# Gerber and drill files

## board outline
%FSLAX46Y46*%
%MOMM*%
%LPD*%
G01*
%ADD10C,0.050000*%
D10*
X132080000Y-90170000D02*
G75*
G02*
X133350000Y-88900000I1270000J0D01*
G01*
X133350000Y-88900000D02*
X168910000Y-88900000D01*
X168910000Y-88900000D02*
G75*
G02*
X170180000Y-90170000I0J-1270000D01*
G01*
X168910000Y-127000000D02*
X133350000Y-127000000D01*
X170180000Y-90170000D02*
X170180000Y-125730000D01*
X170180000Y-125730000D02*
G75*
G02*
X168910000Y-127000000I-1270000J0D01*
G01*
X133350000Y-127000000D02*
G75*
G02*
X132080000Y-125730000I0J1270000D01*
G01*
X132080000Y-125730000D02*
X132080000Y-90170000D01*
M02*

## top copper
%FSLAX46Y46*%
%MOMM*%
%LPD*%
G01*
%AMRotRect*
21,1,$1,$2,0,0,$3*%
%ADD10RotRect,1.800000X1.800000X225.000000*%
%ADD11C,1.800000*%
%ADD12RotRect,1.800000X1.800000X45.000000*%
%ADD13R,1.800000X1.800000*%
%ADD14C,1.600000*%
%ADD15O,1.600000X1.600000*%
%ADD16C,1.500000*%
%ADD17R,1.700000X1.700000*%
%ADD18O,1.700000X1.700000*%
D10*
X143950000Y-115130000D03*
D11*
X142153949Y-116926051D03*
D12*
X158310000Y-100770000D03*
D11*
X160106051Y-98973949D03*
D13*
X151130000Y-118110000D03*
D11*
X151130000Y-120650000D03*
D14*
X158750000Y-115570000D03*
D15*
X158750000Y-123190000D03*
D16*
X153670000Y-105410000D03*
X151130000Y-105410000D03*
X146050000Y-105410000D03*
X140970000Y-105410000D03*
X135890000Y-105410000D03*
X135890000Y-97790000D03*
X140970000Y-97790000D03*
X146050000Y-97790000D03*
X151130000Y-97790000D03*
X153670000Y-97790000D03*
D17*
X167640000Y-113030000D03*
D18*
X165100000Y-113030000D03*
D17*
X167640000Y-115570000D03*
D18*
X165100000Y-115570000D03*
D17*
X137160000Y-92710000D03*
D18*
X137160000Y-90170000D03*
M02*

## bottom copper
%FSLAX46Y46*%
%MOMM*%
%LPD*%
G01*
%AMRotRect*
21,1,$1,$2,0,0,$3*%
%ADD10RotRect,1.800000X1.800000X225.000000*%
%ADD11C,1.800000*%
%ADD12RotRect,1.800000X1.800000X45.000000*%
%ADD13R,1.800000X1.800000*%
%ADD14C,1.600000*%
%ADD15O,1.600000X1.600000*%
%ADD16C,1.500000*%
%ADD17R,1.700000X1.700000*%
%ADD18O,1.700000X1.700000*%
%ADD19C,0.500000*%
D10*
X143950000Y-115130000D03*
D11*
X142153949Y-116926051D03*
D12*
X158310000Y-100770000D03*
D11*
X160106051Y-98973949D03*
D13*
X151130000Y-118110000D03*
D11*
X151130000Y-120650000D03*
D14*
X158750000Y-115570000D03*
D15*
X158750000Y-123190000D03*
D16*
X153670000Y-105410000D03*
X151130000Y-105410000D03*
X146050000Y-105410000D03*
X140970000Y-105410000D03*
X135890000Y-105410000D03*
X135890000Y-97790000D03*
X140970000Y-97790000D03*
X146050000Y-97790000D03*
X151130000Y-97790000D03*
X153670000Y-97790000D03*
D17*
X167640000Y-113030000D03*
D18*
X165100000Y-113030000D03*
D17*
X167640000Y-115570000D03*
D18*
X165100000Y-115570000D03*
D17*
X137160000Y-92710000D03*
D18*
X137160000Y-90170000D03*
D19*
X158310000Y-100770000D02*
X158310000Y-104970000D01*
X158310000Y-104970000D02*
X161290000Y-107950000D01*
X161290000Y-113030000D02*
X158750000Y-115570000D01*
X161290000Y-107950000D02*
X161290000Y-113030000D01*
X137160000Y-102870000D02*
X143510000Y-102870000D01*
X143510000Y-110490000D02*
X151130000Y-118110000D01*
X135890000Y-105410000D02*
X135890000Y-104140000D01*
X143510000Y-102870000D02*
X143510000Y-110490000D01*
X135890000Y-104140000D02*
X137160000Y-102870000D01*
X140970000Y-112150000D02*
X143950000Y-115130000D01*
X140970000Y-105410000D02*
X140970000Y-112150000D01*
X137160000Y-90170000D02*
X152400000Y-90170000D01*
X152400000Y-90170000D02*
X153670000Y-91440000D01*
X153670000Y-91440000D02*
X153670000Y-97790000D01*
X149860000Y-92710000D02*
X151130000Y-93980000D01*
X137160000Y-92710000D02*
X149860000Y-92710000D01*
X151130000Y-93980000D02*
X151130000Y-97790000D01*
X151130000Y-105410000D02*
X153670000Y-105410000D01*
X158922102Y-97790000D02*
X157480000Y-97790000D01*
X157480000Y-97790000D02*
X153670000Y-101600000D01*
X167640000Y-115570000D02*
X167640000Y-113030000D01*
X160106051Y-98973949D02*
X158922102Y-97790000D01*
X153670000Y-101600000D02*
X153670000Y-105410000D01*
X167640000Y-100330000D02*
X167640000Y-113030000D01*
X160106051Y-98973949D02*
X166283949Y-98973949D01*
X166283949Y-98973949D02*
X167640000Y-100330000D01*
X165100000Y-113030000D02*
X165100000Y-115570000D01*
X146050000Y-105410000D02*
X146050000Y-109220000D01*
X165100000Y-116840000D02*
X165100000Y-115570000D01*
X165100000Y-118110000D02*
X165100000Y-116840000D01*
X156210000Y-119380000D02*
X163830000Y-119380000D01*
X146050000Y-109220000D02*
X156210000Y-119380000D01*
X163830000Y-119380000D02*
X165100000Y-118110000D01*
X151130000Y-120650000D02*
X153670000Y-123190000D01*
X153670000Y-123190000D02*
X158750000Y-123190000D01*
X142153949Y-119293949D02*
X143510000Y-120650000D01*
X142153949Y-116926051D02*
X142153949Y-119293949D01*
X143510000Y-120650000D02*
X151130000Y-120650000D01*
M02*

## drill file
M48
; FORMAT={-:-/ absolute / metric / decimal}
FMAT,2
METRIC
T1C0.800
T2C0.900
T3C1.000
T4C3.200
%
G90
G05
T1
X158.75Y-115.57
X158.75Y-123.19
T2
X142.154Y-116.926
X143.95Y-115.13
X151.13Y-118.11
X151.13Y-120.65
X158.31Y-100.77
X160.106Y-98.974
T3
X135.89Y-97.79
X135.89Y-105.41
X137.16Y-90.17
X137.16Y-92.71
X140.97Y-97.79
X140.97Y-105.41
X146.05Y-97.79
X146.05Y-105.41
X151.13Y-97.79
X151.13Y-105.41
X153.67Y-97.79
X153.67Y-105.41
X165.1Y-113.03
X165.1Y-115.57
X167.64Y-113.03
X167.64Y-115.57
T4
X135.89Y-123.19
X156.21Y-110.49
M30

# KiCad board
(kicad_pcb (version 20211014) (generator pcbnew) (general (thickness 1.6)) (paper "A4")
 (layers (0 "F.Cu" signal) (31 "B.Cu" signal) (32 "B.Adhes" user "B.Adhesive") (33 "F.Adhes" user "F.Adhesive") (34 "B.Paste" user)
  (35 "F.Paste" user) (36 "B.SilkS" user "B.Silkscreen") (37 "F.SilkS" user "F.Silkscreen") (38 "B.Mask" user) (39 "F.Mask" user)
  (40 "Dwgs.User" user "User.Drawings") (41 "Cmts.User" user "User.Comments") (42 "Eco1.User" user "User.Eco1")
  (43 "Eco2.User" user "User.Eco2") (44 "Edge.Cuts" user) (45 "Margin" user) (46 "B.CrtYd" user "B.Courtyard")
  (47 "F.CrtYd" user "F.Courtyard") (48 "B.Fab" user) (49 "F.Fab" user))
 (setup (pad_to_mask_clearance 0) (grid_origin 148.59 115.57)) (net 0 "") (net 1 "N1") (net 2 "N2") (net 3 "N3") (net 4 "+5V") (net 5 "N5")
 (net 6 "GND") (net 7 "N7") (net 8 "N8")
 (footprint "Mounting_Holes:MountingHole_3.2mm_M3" (layer "F.Cu") (at 156.21 110.49 -90)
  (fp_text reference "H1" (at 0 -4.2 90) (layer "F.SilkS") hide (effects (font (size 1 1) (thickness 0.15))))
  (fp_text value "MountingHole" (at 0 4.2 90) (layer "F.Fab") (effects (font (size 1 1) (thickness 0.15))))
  (pad "" np_thru_hole circle locked (at 0 0 270) (size 3.2 3.2) (drill 3.2) (layers *.Cu *.Mask) (thermal_gap 2)))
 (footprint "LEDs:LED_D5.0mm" (layer "F.Cu") (at 143.95 115.13 -135)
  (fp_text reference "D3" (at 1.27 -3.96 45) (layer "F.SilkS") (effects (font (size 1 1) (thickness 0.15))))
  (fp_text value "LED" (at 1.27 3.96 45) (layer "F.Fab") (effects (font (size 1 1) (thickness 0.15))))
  (pad "1" thru_hole rect locked (at 0 0 225) (size 1.8 1.8) (drill 0.9) (layers *.Cu *.Mask) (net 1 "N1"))
  (pad "2" thru_hole circle locked (at 2.54 0 225) (size 1.8 1.8) (drill 0.9) (layers *.Cu *.Mask) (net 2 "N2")))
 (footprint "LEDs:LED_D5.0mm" (layer "F.Cu") (at 158.31 100.77 45)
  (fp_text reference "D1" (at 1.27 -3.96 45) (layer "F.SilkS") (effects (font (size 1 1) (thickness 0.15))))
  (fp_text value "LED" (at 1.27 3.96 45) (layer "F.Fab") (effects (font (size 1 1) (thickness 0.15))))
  (pad "1" thru_hole rect locked (at 0 0 45) (size 1.8 1.8) (drill 0.9) (layers *.Cu *.Mask) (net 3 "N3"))
  (pad "2" thru_hole circle locked (at 2.54 0 45) (size 1.8 1.8) (drill 0.9) (layers *.Cu *.Mask) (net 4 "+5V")))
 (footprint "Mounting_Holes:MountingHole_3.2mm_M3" (layer "F.Cu") (at 135.89 123.19 -90)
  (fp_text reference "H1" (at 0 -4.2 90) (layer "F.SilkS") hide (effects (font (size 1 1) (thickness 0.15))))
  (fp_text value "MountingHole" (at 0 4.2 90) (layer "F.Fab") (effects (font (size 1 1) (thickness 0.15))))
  (pad "" np_thru_hole circle locked (at 0 0 270) (size 3.2 3.2) (drill 3.2) (layers *.Cu *.Mask) (thermal_gap 2)))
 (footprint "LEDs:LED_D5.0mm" (layer "F.Cu") (at 151.13 118.11 -90)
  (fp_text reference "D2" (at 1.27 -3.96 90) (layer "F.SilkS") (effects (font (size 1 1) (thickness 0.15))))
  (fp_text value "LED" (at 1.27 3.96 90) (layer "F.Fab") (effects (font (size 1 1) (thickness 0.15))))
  (pad "1" thru_hole rect locked (at 0 0 270) (size 1.8 1.8) (drill 0.9) (layers *.Cu *.Mask) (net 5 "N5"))
  (pad "2" thru_hole circle locked (at 2.54 0 270) (size 1.8 1.8) (drill 0.9) (layers *.Cu *.Mask) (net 2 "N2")))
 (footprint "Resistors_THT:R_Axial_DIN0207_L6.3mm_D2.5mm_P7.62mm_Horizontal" (layer "F.Cu") (at 158.75 115.57 -90)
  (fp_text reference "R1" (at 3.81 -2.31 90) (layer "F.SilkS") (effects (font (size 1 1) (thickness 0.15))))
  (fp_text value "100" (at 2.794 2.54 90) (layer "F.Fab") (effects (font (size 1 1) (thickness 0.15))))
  (pad "1" thru_hole circle locked (at 0 0 270) (size 1.6 1.6) (drill 0.8) (layers *.Cu *.Mask) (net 3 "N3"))
  (pad "2" thru_hole oval locked (at 7.62 0 270) (size 1.6 1.6) (drill 0.8) (layers *.Cu *.Mask) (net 2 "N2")))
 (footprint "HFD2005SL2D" (layer "B.Cu") (at 153.67 105.41 180)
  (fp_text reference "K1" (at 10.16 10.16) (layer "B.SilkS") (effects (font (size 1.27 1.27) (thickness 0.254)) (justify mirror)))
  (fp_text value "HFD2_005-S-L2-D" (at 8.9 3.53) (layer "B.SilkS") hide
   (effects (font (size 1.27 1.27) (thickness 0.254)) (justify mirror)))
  (pad "1" thru_hole circle locked (at 0 0 90) (size 1.5 1.5) (drill 1) (layers *.Cu *.Mask "B.SilkS") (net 4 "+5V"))
  (pad "2" thru_hole circle locked (at 2.54 0 90) (size 1.5 1.5) (drill 1) (layers *.Cu *.Mask "B.SilkS") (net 4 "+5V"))
  (pad "4" thru_hole circle locked (at 7.62 0 90) (size 1.5 1.5) (drill 1) (layers *.Cu *.Mask "B.SilkS") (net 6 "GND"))
  (pad "6" thru_hole circle locked (at 12.7 0 90) (size 1.5 1.5) (drill 1) (layers *.Cu *.Mask "B.SilkS") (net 1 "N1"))
  (pad "8" thru_hole circle locked (at 17.78 0 90) (size 1.5 1.5) (drill 1) (layers *.Cu *.Mask "B.SilkS") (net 5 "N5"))
  (pad "9" thru_hole circle locked (at 17.78 7.62 90) (size 1.5 1.5) (drill 1) (layers *.Cu *.Mask "B.SilkS"))
  (pad "11" thru_hole circle locked (at 12.7 7.62 90) (size 1.5 1.5) (drill 1) (layers *.Cu *.Mask "B.SilkS"))
  (pad "13" thru_hole circle locked (at 7.62 7.62 90) (size 1.5 1.5) (drill 1) (layers *.Cu *.Mask "B.SilkS"))
  (pad "15" thru_hole circle locked (at 2.54 7.62 90) (size 1.5 1.5) (drill 1) (layers *.Cu *.Mask "B.SilkS") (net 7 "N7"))
  (pad "16" thru_hole circle locked (at 0 7.62 90) (size 1.5 1.5) (drill 1) (layers *.Cu *.Mask "B.SilkS") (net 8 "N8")))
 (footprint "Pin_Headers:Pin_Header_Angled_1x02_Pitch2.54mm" (layer "B.Cu") (at 167.64 113.03 90)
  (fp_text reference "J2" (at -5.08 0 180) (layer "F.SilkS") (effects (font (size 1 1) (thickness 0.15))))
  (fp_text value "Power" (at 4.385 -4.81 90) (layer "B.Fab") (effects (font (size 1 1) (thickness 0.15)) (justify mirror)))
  (pad "1" thru_hole rect locked (at 0 0 90) (size 1.7 1.7) (drill 1) (layers *.Cu *.Mask) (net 4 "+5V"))
  (pad "2" thru_hole oval locked (at 0 -2.54 90) (size 1.7 1.7) (drill 1) (layers *.Cu *.Mask) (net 6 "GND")))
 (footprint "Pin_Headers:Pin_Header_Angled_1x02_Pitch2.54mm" (layer "B.Cu") (at 167.64 115.57 90)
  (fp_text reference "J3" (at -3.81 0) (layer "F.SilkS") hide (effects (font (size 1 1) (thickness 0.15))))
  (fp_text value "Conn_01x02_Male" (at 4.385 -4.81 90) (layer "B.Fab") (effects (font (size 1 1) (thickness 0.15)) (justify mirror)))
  (pad "1" thru_hole rect locked (at 0 0 90) (size 1.7 1.7) (drill 1) (layers *.Cu *.Mask) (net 4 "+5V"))
  (pad "2" thru_hole oval locked (at 0 -2.54 90) (size 1.7 1.7) (drill 1) (layers *.Cu *.Mask) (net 6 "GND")))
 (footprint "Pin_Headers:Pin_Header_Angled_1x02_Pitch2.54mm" (layer "B.Cu") (at 137.16 92.71)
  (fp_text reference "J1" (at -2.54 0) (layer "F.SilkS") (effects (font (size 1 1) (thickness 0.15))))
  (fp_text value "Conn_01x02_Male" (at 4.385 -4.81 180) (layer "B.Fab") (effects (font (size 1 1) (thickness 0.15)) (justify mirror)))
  (pad "1" thru_hole rect locked (at 0 0) (size 1.7 1.7) (drill 1) (layers *.Cu *.Mask) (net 7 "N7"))
  (pad "2" thru_hole oval locked (at 0 -2.54) (size 1.7 1.7) (drill 1) (layers *.Cu *.Mask) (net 8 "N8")))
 (gr_arc (start 132.08 90.17) (mid 132.451974 89.271974) (end 133.35 88.9) (layer "Edge.Cuts") (width 0.05))
 (gr_line (start 133.35 88.9) (end 168.91 88.9) (layer "Edge.Cuts") (width 0.05))
 (gr_arc (start 168.91 88.9) (mid 169.808026 89.271974) (end 170.18 90.17) (layer "Edge.Cuts") (width 0.05))
 (gr_line (start 168.91 127) (end 133.35 127) (layer "Edge.Cuts") (width 0.05))
 (gr_line (start 170.18 90.17) (end 170.18 125.73) (layer "Edge.Cuts") (width 0.05))
 (gr_arc (start 170.18 125.73) (mid 169.808026 126.628026) (end 168.91 127) (layer "Edge.Cuts") (width 0.05))
 (gr_arc (start 133.35 127) (mid 132.451974 126.628026) (end 132.08 125.73) (layer "Edge.Cuts") (width 0.05))
 (gr_line (start 132.08 125.73) (end 132.08 90.17) (layer "Edge.Cuts") (width 0.05))
 (segment (start 158.31 100.77) (end 158.31 104.97) (width 0.5) (layer "B.Cu") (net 3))
 (segment (start 158.31 104.97) (end 161.29 107.95) (width 0.5) (layer "B.Cu") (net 3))
 (segment (start 161.29 113.03) (end 158.75 115.57) (width 0.5) (layer "B.Cu") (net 3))
 (segment (start 161.29 107.95) (end 161.29 113.03) (width 0.5) (layer "B.Cu") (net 3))
 (segment (start 137.16 102.87) (end 143.51 102.87) (width 0.5) (layer "B.Cu") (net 5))
 (segment (start 143.51 110.49) (end 151.13 118.11) (width 0.5) (layer "B.Cu") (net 5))
 (segment (start 135.89 105.41) (end 135.89 104.14) (width 0.5) (layer "B.Cu") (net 5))
 (segment (start 143.51 102.87) (end 143.51 110.49) (width 0.5) (layer "B.Cu") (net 5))
 (segment (start 135.89 104.14) (end 137.16 102.87) (width 0.5) (layer "B.Cu") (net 5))
 (segment (start 140.97 112.15) (end 143.95 115.13) (width 0.5) (layer "B.Cu") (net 1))
 (segment (start 140.97 105.41) (end 140.97 112.15) (width 0.5) (layer "B.Cu") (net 1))
 (segment (start 137.16 90.17) (end 152.4 90.17) (width 0.5) (layer "B.Cu") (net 8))
 (segment (start 152.4 90.17) (end 153.67 91.44) (width 0.5) (layer "B.Cu") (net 8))
 (segment (start 153.67 91.44) (end 153.67 97.79) (width 0.5) (layer "B.Cu") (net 8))
 (segment (start 149.86 92.71) (end 151.13 93.98) (width 0.5) (layer "B.Cu") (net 7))
 (segment (start 137.16 92.71) (end 149.86 92.71) (width 0.5) (layer "B.Cu") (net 7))
 (segment (start 151.13 93.98) (end 151.13 97.79) (width 0.5) (layer "B.Cu") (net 7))
 (segment (start 151.13 105.41) (end 153.67 105.41) (width 0.5) (layer "B.Cu") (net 4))
 (segment (start 158.922102 97.79) (end 157.48 97.79) (width 0.5) (layer "B.Cu") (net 4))
 (segment (start 157.48 97.79) (end 153.67 101.6) (width 0.5) (layer "B.Cu") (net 4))
 (segment (start 167.64 115.57) (end 167.64 113.03) (width 0.5) (layer "B.Cu") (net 4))
 (segment (start 160.106051 98.973949) (end 158.922102 97.79) (width 0.5) (layer "B.Cu") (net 4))
 (segment (start 153.67 101.6) (end 153.67 105.41) (width 0.5) (layer "B.Cu") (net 4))
 (segment (start 167.64 100.33) (end 167.64 113.03) (width 0.5) (layer "B.Cu") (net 4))
 (segment (start 160.106051 98.973949) (end 166.283949 98.973949) (width 0.5) (layer "B.Cu") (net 4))
 (segment (start 166.283949 98.973949) (end 167.64 100.33) (width 0.5) (layer "B.Cu") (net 4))
 (segment (start 165.1 113.03) (end 165.1 115.57) (width 0.5) (layer "B.Cu") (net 6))
 (segment (start 146.05 105.41) (end 146.05 109.22) (width 0.5) (layer "B.Cu") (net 6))
 (segment (start 165.1 116.84) (end 165.1 115.57) (width 0.5) (layer "B.Cu") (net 6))
 (segment (start 165.1 118.11) (end 165.1 116.84) (width 0.5) (layer "B.Cu") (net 6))
 (segment (start 156.21 119.38) (end 163.83 119.38) (width 0.5) (layer "B.Cu") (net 6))
 (segment (start 146.05 109.22) (end 156.21 119.38) (width 0.5) (layer "B.Cu") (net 6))
 (segment (start 163.83 119.38) (end 165.1 118.11) (width 0.5) (layer "B.Cu") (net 6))
 (segment (start 151.13 120.65) (end 153.67 123.19) (width 0.5) (layer "B.Cu") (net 2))
 (segment (start 153.67 123.19) (end 158.75 123.19) (width 0.5) (layer "B.Cu") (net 2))
 (segment (start 142.153949 119.293949) (end 143.51 120.65) (width 0.5) (layer "B.Cu") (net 2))
 (segment (start 142.153949 116.926051) (end 142.153949 119.293949) (width 0.5) (layer "B.Cu") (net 2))
 (segment (start 143.51 120.65) (end 151.13 120.65) (width 0.5) (layer "B.Cu") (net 2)))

